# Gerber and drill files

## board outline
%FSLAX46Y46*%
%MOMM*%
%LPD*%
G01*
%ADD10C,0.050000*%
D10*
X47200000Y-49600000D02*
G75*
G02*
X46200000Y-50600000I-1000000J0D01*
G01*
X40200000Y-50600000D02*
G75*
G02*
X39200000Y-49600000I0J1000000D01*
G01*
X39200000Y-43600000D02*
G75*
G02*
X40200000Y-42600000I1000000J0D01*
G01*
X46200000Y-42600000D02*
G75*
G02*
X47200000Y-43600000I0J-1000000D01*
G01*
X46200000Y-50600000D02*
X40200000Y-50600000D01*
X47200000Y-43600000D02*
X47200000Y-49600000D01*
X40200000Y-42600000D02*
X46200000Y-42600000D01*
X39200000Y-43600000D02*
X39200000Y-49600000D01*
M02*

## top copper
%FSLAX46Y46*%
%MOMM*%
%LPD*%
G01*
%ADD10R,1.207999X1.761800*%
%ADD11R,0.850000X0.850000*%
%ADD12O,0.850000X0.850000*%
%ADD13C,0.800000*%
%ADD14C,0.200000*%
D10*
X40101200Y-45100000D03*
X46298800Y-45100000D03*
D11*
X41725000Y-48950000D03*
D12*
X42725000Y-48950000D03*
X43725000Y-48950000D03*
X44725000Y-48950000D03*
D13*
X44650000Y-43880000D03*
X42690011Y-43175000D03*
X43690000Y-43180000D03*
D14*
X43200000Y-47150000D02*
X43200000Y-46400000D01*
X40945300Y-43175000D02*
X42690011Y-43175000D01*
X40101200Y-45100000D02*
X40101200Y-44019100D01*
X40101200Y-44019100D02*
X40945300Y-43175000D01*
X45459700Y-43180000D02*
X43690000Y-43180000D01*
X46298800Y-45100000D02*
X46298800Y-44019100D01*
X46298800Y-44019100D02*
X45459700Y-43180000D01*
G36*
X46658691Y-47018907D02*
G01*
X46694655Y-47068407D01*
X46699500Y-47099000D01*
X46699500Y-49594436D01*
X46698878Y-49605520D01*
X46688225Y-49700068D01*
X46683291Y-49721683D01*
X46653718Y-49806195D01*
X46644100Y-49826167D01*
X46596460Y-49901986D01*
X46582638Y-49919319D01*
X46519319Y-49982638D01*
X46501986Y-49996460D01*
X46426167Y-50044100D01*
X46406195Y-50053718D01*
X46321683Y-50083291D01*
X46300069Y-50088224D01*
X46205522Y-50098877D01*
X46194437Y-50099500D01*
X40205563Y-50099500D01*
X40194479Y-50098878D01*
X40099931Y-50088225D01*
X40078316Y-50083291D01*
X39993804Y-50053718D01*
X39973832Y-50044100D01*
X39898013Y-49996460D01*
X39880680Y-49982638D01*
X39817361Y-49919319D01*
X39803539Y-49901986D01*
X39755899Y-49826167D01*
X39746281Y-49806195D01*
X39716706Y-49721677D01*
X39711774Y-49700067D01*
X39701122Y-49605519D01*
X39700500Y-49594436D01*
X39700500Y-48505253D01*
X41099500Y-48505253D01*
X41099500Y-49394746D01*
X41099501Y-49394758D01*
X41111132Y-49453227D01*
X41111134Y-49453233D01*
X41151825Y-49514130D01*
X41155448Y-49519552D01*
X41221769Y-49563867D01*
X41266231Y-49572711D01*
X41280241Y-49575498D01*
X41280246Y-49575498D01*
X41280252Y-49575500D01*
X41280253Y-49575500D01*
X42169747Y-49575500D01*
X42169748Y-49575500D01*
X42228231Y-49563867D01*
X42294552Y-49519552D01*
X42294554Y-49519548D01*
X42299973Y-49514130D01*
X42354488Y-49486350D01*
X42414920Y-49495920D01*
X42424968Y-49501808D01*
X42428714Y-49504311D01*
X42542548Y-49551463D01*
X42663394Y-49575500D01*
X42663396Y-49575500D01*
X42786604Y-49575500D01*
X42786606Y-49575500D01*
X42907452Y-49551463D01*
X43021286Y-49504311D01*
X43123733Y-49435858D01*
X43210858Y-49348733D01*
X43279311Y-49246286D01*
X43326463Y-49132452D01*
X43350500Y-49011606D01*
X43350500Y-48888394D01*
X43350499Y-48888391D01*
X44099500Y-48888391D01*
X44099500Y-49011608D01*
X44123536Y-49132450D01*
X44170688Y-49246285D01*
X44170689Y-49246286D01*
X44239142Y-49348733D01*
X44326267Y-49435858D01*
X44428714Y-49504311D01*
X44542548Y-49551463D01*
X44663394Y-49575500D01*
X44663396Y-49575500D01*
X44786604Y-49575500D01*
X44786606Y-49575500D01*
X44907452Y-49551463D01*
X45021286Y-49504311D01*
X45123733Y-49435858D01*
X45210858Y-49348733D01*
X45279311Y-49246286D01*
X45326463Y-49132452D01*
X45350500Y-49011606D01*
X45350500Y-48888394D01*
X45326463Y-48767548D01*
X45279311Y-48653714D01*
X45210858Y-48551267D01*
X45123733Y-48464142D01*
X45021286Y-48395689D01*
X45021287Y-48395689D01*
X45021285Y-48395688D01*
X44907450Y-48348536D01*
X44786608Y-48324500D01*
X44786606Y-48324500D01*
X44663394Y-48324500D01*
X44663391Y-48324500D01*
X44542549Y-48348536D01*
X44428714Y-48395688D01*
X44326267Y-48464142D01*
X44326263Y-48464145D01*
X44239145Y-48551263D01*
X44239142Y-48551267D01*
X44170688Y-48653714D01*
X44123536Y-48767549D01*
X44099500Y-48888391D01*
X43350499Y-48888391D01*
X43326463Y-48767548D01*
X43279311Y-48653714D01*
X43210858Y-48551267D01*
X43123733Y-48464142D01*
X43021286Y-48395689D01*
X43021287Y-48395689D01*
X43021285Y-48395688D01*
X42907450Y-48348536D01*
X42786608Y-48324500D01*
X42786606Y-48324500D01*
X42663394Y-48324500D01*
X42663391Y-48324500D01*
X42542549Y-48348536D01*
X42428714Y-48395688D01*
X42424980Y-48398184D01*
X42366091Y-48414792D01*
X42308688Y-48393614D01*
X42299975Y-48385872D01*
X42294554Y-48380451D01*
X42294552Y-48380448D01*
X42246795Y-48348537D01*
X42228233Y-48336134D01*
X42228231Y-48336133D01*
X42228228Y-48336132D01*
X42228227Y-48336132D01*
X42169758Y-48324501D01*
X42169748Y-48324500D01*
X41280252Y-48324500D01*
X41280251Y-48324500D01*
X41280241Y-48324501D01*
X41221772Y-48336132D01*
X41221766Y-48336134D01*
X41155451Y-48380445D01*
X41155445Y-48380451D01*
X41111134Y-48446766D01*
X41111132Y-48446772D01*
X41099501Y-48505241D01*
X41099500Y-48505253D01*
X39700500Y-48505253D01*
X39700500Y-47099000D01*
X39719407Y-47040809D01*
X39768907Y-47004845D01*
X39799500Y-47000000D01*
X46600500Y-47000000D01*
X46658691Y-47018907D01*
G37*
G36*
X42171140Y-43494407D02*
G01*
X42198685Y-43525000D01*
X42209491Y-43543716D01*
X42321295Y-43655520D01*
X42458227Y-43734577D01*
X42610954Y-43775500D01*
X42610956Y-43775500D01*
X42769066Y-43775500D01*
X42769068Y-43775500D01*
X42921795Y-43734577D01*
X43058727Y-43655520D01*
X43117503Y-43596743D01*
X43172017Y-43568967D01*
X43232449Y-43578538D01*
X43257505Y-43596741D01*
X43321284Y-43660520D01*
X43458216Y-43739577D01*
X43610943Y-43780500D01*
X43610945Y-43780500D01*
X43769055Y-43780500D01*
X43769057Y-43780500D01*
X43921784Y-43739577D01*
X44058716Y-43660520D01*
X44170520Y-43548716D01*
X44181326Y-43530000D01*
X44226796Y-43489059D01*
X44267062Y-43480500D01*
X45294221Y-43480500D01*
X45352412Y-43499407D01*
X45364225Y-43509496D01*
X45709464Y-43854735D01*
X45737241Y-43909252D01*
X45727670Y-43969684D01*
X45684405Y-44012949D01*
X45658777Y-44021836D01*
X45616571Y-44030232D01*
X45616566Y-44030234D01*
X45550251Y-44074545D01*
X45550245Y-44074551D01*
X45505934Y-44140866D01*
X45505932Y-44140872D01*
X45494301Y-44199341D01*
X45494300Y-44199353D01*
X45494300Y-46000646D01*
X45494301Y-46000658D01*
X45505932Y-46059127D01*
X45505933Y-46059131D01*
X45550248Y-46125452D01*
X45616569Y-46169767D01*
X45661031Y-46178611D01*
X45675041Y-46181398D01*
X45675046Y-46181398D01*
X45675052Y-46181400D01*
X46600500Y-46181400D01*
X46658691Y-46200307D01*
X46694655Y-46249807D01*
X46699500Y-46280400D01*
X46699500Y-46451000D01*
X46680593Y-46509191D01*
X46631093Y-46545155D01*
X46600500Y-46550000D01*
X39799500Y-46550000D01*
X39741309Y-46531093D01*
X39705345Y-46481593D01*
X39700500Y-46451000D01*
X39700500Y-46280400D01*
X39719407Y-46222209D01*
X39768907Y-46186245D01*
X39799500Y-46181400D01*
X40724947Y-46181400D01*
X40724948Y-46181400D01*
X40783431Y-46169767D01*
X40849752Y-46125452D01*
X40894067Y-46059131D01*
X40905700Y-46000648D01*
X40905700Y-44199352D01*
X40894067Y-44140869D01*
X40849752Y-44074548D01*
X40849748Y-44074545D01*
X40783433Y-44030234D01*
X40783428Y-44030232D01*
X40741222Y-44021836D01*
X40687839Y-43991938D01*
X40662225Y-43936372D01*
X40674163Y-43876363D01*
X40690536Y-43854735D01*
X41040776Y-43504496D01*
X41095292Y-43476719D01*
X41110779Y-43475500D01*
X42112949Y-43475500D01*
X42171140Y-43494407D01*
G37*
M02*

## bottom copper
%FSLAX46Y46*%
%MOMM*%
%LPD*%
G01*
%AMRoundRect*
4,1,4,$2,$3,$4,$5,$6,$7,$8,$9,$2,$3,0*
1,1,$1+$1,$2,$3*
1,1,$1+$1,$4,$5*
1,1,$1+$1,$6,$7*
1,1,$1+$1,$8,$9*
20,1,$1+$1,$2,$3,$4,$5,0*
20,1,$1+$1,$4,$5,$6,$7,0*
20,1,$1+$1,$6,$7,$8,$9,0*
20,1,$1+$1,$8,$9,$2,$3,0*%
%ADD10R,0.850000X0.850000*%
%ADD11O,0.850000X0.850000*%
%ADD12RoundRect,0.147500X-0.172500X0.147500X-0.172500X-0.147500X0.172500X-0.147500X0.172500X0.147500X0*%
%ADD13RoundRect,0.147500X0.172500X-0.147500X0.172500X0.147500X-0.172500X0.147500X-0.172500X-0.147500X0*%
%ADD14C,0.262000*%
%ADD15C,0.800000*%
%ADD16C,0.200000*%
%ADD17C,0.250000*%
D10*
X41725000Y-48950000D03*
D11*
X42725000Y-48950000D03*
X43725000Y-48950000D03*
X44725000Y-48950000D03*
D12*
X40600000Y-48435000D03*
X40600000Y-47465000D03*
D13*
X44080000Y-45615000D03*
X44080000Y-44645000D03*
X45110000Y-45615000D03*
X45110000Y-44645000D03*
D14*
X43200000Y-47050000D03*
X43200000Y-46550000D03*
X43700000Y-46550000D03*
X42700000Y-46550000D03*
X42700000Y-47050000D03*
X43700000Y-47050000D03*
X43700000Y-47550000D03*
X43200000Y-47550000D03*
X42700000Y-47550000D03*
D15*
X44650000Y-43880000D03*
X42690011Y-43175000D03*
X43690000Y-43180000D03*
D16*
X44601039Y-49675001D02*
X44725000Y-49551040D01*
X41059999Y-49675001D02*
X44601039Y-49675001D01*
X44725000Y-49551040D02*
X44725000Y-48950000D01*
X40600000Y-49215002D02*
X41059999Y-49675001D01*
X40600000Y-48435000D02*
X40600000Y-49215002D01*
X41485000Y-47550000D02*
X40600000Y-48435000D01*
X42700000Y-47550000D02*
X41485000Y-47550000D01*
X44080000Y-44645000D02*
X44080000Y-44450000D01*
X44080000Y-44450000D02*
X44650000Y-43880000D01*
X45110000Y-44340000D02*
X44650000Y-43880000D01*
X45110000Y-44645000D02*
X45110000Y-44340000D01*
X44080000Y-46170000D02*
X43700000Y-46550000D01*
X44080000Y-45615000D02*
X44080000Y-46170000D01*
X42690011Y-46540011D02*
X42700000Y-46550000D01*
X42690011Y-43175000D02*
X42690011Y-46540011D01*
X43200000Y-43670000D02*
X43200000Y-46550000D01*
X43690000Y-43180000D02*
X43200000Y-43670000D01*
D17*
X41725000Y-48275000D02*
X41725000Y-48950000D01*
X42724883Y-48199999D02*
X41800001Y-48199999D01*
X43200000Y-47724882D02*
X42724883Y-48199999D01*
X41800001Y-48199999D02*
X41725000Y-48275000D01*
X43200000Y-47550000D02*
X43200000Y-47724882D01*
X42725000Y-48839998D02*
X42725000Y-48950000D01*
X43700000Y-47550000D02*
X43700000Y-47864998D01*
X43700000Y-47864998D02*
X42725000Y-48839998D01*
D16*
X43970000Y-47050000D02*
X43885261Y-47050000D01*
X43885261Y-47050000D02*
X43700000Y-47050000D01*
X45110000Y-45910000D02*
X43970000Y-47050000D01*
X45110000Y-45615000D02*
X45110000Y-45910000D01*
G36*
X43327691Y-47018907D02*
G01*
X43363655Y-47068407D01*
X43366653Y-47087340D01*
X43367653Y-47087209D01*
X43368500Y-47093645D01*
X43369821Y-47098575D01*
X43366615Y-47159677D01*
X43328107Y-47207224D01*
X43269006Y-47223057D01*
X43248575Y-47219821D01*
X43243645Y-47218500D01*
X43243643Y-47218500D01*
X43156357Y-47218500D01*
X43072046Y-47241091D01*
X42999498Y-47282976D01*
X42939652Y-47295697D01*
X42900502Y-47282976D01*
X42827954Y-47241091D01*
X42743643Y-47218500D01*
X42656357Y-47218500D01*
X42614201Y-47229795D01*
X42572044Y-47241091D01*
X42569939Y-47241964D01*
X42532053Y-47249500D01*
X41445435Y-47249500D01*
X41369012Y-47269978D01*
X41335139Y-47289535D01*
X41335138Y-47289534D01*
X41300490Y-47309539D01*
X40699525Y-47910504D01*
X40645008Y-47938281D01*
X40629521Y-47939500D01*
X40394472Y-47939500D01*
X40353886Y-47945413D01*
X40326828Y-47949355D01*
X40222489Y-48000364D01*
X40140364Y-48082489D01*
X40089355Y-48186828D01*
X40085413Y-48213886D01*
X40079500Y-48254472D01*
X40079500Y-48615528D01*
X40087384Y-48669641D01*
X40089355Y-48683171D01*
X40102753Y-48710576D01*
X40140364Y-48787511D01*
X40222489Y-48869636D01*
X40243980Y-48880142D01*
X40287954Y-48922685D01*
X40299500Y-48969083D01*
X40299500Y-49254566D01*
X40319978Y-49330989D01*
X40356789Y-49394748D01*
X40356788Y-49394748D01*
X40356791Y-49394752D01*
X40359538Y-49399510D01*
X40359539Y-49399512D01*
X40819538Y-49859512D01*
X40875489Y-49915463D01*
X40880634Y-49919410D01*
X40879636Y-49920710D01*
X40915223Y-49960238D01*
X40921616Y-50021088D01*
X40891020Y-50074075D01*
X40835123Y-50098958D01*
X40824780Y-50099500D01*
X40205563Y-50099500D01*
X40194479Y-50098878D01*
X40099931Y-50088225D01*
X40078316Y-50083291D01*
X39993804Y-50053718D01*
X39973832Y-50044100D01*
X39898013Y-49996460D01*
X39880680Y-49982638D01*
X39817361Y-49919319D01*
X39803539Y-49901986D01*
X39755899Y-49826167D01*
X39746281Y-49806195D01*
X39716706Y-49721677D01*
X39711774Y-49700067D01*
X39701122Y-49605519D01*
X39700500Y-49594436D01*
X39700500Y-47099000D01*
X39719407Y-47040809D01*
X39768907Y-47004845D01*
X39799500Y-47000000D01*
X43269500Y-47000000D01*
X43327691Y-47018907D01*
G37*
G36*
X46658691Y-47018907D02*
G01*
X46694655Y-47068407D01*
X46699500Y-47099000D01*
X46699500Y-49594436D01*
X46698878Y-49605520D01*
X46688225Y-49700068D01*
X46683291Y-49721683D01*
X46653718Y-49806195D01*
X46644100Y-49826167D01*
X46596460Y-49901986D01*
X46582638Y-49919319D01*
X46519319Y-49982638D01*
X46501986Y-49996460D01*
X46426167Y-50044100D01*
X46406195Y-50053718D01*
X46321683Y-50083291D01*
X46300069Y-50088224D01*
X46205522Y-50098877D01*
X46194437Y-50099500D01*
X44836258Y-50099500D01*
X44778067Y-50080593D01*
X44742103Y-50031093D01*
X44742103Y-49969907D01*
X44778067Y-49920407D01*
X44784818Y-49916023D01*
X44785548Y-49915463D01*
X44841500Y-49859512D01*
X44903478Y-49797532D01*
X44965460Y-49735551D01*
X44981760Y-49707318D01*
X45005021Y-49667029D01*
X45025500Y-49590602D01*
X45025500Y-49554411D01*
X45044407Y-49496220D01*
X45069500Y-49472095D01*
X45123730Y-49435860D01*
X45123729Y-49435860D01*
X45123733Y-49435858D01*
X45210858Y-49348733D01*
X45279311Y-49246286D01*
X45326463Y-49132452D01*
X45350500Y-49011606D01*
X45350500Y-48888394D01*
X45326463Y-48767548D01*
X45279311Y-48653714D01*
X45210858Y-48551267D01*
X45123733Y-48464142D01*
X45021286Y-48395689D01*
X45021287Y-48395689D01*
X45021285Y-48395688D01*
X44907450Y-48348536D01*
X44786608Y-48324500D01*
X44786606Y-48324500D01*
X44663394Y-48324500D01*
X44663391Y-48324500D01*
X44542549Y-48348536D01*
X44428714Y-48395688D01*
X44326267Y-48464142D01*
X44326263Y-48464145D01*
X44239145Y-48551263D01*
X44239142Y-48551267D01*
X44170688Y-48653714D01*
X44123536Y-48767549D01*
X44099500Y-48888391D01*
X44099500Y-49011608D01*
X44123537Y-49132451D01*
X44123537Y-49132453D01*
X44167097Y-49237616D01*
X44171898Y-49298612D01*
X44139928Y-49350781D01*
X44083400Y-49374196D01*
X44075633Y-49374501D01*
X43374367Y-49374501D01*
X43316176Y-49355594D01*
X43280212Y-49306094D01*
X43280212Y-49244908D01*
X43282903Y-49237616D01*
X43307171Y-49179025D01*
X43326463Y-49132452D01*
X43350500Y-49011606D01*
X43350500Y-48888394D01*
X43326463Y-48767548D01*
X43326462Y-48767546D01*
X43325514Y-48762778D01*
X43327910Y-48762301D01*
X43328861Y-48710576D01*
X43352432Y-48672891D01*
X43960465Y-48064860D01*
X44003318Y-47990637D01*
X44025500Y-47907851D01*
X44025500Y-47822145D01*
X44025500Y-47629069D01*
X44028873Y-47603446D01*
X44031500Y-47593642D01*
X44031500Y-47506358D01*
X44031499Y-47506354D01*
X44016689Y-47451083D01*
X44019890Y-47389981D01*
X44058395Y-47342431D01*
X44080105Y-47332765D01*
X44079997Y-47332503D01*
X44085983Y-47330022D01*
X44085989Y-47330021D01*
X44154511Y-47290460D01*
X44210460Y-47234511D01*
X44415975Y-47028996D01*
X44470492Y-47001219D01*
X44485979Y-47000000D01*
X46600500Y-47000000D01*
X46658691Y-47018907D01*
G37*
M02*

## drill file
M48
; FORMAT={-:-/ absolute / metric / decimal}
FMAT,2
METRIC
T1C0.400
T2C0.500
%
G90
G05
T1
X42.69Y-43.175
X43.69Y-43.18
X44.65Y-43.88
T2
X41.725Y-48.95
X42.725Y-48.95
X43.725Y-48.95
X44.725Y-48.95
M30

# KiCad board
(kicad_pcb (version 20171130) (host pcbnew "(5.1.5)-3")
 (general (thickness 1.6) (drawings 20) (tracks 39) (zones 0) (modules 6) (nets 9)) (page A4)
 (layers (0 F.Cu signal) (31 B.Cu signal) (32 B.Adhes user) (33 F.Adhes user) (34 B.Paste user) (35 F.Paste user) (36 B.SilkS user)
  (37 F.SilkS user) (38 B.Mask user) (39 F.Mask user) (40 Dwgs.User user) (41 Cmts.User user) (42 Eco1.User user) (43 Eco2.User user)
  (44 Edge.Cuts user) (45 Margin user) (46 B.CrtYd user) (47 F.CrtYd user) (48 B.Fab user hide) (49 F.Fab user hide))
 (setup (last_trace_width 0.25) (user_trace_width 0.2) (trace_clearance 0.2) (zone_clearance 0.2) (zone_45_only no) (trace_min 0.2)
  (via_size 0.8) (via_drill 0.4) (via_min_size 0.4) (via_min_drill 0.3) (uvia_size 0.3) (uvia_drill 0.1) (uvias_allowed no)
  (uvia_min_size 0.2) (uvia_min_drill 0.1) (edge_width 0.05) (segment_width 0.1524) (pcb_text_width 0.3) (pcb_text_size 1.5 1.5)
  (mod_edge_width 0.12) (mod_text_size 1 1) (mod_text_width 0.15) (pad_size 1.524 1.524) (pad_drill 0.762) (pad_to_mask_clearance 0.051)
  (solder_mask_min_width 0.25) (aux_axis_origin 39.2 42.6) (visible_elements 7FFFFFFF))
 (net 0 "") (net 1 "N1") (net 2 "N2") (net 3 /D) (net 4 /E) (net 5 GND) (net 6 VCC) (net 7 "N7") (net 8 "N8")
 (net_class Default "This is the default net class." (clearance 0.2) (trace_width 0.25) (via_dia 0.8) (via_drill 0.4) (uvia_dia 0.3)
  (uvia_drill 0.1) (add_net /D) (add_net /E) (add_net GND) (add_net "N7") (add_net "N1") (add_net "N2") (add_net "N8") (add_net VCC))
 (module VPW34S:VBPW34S (layer F.Cu) (at 43.2 45.1)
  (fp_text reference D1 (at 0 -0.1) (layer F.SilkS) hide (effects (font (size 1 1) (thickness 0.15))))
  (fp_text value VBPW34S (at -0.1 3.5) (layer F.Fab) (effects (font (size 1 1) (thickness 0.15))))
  (pad 1 smd rect (at -3.0988 0) (size 1.207999 1.7618) (layers F.Cu F.Paste F.Mask) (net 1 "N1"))
  (pad 2 smd rect (at 3.0988 0) (size 1.207999 1.7618) (layers F.Cu F.Paste F.Mask) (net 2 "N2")))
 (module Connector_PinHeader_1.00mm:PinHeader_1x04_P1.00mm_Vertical (layer F.Cu) (at 41.725 48.95 90)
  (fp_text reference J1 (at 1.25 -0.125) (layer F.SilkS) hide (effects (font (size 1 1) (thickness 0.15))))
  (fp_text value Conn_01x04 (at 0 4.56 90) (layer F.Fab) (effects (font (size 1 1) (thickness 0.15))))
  (pad 1 thru_hole rect (at 0 0 90) (size 0.85 0.85) (drill 0.5) (layers *.Cu *.Mask) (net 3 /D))
  (pad 2 thru_hole oval (at 0 1 90) (size 0.85 0.85) (drill 0.5) (layers *.Cu *.Mask) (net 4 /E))
  (pad 3 thru_hole oval (at 0 2 90) (size 0.85 0.85) (drill 0.5) (layers *.Cu *.Mask) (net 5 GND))
  (pad 4 thru_hole oval (at 0 3 90) (size 0.85 0.85) (drill 0.5) (layers *.Cu *.Mask) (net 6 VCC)))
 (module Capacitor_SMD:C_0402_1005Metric (layer B.Cu) (at 40.6 47.95 270)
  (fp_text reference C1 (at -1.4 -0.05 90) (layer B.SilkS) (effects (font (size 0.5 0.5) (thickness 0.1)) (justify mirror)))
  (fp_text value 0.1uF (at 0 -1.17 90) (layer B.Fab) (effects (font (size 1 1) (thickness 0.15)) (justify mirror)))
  (pad 2 smd roundrect (at 0.485 0 270) (size 0.59 0.64) (layers B.Cu B.Paste B.Mask) (roundrect_rratio 0.25) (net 6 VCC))
  (pad 1 smd roundrect (at -0.485 0 270) (size 0.59 0.64) (layers B.Cu B.Paste B.Mask) (roundrect_rratio 0.25) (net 5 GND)))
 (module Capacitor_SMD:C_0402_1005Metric (layer B.Cu) (at 44.08 45.13 90)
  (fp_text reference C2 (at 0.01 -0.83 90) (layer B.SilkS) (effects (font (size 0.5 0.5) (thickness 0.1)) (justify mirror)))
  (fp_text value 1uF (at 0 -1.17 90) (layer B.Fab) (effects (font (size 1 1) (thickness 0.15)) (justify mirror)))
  (pad 1 smd roundrect (at -0.485 0 90) (size 0.59 0.64) (layers B.Cu B.Paste B.Mask) (roundrect_rratio 0.25) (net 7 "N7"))
  (pad 2 smd roundrect (at 0.485 0 90) (size 0.59 0.64) (layers B.Cu B.Paste B.Mask) (roundrect_rratio 0.25) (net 5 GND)))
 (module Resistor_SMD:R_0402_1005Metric (layer B.Cu) (at 45.11 45.13 90)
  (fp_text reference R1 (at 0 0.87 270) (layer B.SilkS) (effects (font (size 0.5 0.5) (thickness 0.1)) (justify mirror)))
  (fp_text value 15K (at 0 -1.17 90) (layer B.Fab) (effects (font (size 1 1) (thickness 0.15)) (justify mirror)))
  (pad 1 smd roundrect (at -0.485 0 90) (size 0.59 0.64) (layers B.Cu B.Paste B.Mask) (roundrect_rratio 0.25) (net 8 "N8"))
  (pad 2 smd roundrect (at 0.485 0 90) (size 0.59 0.64) (layers B.Cu B.Paste B.Mask) (roundrect_rratio 0.25) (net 5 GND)))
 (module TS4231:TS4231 (layer B.Cu) (at 43.2 47.05 180)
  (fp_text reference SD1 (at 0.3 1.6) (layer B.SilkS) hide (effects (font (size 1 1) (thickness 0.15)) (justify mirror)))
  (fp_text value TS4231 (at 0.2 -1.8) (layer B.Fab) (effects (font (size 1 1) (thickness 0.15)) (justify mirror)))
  (pad B2 smd circle (at 0 0 180) (size 0.262 0.262) (layers B.Cu B.Paste B.Mask) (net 5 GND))
  (pad A2 smd circle (at 0 0.5 180) (size 0.262 0.262) (layers B.Cu B.Paste B.Mask) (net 2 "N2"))
  (pad A1 smd circle (at -0.5 0.5 180) (size 0.262 0.262) (layers B.Cu B.Paste B.Mask) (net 7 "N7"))
  (pad A3 smd circle (at 0.5 0.5 180) (size 0.262 0.262) (layers B.Cu B.Paste B.Mask) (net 1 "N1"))
  (pad B3 smd circle (at 0.5 0 180) (size 0.262 0.262) (layers B.Cu B.Paste B.Mask) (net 5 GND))
  (pad B1 smd circle (at -0.5 0 180) (size 0.262 0.262) (layers B.Cu B.Paste B.Mask) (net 8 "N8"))
  (pad C1 smd circle (at -0.5 -0.5 180) (size 0.262 0.262) (layers B.Cu B.Paste B.Mask) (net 4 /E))
  (pad C2 smd circle (at 0 -0.5 180) (size 0.262 0.262) (layers B.Cu B.Paste B.Mask) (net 3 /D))
  (pad C3 smd circle (at 0.5 -0.5 180) (size 0.262 0.262) (layers B.Cu B.Paste B.Mask) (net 6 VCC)))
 (gr_arc (start 46.2 49.6) (end 46.2 50.6) (angle -90) (layer Edge.Cuts) (width 0.05))
 (gr_arc (start 40.2 49.6) (end 39.2 49.6) (angle -90) (layer Edge.Cuts) (width 0.05))
 (gr_arc (start 40.2 43.6) (end 40.2 42.6) (angle -90) (layer Edge.Cuts) (width 0.05))
 (gr_arc (start 46.2 43.6) (end 47.2 43.6) (angle -90) (layer Edge.Cuts) (width 0.05))
 (gr_line (start 46.2 50.6) (end 40.2 50.6) (layer Edge.Cuts) (width 0.05))
 (gr_line (start 47.2 43.6) (end 47.2 49.6) (layer Edge.Cuts) (width 0.05))
 (gr_line (start 40.2 42.6) (end 46.2 42.6) (layer Edge.Cuts) (width 0.05))
 (gr_line (start 39.2 43.6) (end 39.2 49.6) (layer Edge.Cuts) (width 0.05))
 (segment (start 44.601039 49.675001) (end 44.725 49.55104) (width 0.2) (layer B.Cu) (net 6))
 (segment (start 41.059999 49.675001) (end 44.601039 49.675001) (width 0.2) (layer B.Cu) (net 6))
 (segment (start 44.725 49.55104) (end 44.725 48.95) (width 0.2) (layer B.Cu) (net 6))
 (segment (start 40.6 49.215002) (end 41.059999 49.675001) (width 0.2) (layer B.Cu) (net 6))
 (segment (start 40.6 48.435) (end 40.6 49.215002) (width 0.2) (layer B.Cu) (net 6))
 (segment (start 41.485 47.55) (end 40.6 48.435) (width 0.2) (layer B.Cu) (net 6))
 (segment (start 42.7 47.55) (end 41.485 47.55) (width 0.2) (layer B.Cu) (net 6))
 (segment (start 43.2 47.15) (end 43.2 46.4) (width 0.2) (layer F.Cu) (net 5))
 (via (at 44.65 43.88) (size 0.8) (drill 0.4) (layers F.Cu B.Cu) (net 5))
 (segment (start 44.08 44.645) (end 44.08 44.45) (width 0.2) (layer B.Cu) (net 5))
 (segment (start 44.08 44.45) (end 44.65 43.88) (width 0.2) (layer B.Cu) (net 5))
 (segment (start 45.11 44.34) (end 44.65 43.88) (width 0.2) (layer B.Cu) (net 5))
 (segment (start 45.11 44.645) (end 45.11 44.34) (width 0.2) (layer B.Cu) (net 5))
 (segment (start 44.08 46.17) (end 43.7 46.55) (width 0.2) (layer B.Cu) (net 7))
 (segment (start 44.08 45.615) (end 44.08 46.17) (width 0.2) (layer B.Cu) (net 7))
 (via (at 42.690011 43.175) (size 0.8) (drill 0.4) (layers F.Cu B.Cu) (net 1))
 (segment (start 40.9453 43.175) (end 42.690011 43.175) (width 0.2) (layer F.Cu) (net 1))
 (segment (start 40.1012 45.1) (end 40.1012 44.0191) (width 0.2) (layer F.Cu) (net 1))
 (segment (start 40.1012 44.0191) (end 40.9453 43.175) (width 0.2) (layer F.Cu) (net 1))
 (segment (start 42.690011 46.540011) (end 42.7 46.55) (width 0.2) (layer B.Cu) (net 1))
 (segment (start 42.690011 43.175) (end 42.690011 46.540011) (width 0.2) (layer B.Cu) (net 1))
 (via (at 43.69 43.18) (size 0.8) (drill 0.4) (layers F.Cu B.Cu) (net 2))
 (segment (start 45.4597 43.18) (end 43.69 43.18) (width 0.2) (layer F.Cu) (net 2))
 (segment (start 46.2988 45.1) (end 46.2988 44.0191) (width 0.2) (layer F.Cu) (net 2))
 (segment (start 46.2988 44.0191) (end 45.4597 43.18) (width 0.2) (layer F.Cu) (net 2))
 (segment (start 43.2 43.67) (end 43.2 46.55) (width 0.2) (layer B.Cu) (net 2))
 (segment (start 43.69 43.18) (end 43.2 43.67) (width 0.2) (layer B.Cu) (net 2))
 (segment (start 41.725 48.275) (end 41.725 48.95) (width 0.25) (layer B.Cu) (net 3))
 (segment (start 42.724883 48.199999) (end 41.800001 48.199999) (width 0.25) (layer B.Cu) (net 3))
 (segment (start 43.2 47.724882) (end 42.724883 48.199999) (width 0.25) (layer B.Cu) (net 3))
 (segment (start 41.800001 48.199999) (end 41.725 48.275) (width 0.25) (layer B.Cu) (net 3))
 (segment (start 43.2 47.55) (end 43.2 47.724882) (width 0.25) (layer B.Cu) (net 3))
 (segment (start 42.725 48.839998) (end 42.725 48.95) (width 0.25) (layer B.Cu) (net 4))
 (segment (start 43.7 47.55) (end 43.7 47.864998) (width 0.25) (layer B.Cu) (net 4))
 (segment (start 43.7 47.864998) (end 42.725 48.839998) (width 0.25) (layer B.Cu) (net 4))
 (segment (start 43.97 47.05) (end 43.885261 47.05) (width 0.2) (layer B.Cu) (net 8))
 (segment (start 43.885261 47.05) (end 43.7 47.05) (width 0.2) (layer B.Cu) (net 8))
 (segment (start 45.11 45.91) (end 43.97 47.05) (width 0.2) (layer B.Cu) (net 8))
 (segment (start 45.11 45.615) (end 45.11 45.91) (width 0.2) (layer B.Cu) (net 8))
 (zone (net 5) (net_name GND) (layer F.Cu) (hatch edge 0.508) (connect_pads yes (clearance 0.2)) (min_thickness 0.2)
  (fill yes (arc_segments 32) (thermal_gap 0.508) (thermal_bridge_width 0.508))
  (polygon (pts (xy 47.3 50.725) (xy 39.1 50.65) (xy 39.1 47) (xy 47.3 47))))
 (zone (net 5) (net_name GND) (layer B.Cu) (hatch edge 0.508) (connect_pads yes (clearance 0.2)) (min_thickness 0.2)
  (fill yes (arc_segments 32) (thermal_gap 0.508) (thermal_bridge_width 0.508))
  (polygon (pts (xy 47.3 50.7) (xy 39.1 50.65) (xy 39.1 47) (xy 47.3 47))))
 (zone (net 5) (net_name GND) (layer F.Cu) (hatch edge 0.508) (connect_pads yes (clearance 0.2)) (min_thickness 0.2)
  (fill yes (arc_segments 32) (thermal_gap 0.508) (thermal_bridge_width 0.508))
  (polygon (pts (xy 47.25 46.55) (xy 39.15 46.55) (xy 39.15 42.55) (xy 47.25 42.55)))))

